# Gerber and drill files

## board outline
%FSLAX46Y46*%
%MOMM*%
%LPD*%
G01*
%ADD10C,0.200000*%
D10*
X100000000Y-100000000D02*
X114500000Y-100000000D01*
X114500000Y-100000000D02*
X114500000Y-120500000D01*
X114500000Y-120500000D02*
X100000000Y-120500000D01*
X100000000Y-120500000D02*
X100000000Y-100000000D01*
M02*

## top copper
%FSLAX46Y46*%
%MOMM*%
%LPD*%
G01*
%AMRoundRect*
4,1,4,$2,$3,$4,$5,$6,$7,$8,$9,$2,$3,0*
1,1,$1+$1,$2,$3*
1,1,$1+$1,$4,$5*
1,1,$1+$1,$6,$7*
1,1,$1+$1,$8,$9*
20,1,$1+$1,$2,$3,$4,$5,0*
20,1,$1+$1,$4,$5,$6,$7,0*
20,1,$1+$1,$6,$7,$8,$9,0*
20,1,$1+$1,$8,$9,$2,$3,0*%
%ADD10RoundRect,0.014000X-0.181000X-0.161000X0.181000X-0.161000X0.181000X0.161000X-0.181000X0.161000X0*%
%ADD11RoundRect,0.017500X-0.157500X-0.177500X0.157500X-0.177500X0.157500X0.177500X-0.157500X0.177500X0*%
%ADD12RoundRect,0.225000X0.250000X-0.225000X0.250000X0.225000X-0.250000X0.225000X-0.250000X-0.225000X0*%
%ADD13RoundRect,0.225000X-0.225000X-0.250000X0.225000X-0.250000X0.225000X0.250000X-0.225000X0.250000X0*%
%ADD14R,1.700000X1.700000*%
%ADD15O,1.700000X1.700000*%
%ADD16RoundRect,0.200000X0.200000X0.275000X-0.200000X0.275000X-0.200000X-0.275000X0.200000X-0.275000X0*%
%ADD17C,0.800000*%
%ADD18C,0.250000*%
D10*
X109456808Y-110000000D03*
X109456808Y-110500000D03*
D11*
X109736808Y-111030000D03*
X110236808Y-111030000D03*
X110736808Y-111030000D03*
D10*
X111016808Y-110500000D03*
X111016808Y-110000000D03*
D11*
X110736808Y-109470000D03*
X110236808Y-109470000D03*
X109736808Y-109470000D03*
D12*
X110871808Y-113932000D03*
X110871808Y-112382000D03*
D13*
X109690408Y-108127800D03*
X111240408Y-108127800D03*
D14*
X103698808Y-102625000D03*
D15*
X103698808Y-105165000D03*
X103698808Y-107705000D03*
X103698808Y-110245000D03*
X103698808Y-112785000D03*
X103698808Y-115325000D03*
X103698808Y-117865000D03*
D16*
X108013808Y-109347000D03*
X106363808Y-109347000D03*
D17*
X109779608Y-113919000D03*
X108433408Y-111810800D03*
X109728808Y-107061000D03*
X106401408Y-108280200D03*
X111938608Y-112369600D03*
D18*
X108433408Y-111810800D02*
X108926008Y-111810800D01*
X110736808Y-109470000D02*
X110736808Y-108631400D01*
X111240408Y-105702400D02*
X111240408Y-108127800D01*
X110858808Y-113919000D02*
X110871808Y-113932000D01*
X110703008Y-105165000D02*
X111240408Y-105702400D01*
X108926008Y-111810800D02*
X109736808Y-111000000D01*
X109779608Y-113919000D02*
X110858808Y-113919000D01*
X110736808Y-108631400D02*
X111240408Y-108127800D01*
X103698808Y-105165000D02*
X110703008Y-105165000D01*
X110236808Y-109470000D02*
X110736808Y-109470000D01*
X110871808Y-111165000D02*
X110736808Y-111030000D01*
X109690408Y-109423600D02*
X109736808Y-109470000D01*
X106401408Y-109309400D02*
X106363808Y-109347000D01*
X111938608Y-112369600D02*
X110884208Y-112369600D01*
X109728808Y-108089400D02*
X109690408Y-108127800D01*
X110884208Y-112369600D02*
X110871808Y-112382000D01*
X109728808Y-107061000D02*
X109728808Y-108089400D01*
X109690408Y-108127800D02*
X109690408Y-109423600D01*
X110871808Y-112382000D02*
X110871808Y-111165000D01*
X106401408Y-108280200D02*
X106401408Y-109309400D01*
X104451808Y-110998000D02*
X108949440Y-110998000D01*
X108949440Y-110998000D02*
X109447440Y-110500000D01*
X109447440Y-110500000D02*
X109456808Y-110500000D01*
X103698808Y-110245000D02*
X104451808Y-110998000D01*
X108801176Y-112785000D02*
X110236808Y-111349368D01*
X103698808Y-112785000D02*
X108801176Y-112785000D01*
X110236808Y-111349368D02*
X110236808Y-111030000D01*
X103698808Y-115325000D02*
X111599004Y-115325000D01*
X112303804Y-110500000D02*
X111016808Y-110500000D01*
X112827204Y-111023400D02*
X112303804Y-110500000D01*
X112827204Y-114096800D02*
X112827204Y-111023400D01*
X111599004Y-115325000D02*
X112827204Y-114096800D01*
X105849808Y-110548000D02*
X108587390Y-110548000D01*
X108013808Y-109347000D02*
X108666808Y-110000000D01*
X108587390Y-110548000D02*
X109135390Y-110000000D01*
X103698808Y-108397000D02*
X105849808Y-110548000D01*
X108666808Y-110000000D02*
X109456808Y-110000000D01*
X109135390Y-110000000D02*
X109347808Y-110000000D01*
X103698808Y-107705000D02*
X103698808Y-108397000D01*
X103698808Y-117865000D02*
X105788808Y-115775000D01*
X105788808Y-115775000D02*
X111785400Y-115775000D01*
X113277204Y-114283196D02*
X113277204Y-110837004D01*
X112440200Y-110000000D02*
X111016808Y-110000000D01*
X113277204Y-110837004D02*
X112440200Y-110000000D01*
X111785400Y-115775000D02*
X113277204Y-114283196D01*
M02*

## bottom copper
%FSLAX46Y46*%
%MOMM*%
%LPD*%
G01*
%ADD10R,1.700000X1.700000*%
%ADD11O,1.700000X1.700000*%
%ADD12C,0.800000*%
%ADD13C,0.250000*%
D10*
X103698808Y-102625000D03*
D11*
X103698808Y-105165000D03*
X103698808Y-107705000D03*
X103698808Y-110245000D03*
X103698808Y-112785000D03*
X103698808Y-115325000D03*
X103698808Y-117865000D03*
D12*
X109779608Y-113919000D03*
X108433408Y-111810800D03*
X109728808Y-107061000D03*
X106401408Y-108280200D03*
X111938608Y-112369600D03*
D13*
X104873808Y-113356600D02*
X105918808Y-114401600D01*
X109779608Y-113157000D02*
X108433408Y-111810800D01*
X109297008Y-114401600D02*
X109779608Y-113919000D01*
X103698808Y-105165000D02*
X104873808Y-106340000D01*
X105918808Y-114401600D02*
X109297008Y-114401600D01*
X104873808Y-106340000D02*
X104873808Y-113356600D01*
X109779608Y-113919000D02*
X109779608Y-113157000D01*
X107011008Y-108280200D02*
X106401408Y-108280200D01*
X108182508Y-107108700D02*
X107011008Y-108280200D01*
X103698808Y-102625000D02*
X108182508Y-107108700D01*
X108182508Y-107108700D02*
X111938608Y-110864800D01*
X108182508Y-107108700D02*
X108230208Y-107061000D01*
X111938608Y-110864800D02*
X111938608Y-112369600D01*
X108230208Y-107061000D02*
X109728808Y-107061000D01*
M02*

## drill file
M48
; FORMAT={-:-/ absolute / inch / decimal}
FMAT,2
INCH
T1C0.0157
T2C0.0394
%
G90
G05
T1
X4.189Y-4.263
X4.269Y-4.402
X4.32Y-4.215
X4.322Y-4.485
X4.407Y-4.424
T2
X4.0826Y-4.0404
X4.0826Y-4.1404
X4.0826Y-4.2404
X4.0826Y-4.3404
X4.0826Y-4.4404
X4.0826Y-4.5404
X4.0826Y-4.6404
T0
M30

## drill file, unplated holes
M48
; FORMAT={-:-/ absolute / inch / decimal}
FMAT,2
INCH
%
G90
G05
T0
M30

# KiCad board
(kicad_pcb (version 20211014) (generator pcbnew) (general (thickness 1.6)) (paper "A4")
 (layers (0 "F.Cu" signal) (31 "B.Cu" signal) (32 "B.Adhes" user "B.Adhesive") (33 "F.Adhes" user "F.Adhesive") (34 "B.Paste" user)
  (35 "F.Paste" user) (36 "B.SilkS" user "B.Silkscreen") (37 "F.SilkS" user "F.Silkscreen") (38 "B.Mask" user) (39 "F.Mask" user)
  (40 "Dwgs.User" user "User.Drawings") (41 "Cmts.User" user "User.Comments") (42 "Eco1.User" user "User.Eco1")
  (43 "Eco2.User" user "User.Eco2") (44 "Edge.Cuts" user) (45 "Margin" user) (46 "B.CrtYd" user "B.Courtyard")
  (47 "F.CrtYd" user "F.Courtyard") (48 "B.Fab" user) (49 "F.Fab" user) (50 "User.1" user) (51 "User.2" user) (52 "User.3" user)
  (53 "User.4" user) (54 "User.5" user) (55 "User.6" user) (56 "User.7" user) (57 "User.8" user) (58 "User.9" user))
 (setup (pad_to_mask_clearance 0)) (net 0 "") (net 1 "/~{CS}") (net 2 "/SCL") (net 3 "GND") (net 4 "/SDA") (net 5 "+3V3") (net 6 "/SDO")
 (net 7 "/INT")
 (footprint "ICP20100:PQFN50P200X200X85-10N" (layer "F.Cu") (at 110.236808 110.25)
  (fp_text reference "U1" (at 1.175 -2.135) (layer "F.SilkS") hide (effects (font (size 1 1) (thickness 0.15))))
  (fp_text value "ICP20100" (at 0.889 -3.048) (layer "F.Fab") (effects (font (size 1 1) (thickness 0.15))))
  (pad "1" smd roundrect locked (at -0.78 -0.25) (size 0.39 0.35) (layers "F.Cu" "F.Paste" "F.Mask") (roundrect_rratio 0.04)
   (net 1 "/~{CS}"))
  (pad "2" smd roundrect locked (at -0.78 0.25) (size 0.39 0.35) (layers "F.Cu" "F.Paste" "F.Mask") (roundrect_rratio 0.04) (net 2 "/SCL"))
  (pad "3" smd roundrect locked (at -0.5 0.78) (size 0.35 0.39) (layers "F.Cu" "F.Paste" "F.Mask") (roundrect_rratio 0.05) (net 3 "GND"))
  (pad "4" smd roundrect locked (at 0 0.78) (size 0.35 0.39) (layers "F.Cu" "F.Paste" "F.Mask") (roundrect_rratio 0.05) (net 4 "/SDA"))
  (pad "5" smd roundrect locked (at 0.5 0.78) (size 0.35 0.39) (layers "F.Cu" "F.Paste" "F.Mask") (roundrect_rratio 0.05) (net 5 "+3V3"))
  (pad "6" smd roundrect locked (at 0.78 0.25) (size 0.39 0.35) (layers "F.Cu" "F.Paste" "F.Mask") (roundrect_rratio 0.04) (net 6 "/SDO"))
  (pad "7" smd roundrect locked (at 0.78 -0.25) (size 0.39 0.35) (layers "F.Cu" "F.Paste" "F.Mask") (roundrect_rratio 0.04) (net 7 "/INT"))
  (pad "8" smd roundrect locked (at 0.5 -0.78) (size 0.35 0.39) (layers "F.Cu" "F.Paste" "F.Mask") (roundrect_rratio 0.05) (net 3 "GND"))
  (pad "9" smd roundrect locked (at 0 -0.78) (size 0.35 0.39) (layers "F.Cu" "F.Paste" "F.Mask") (roundrect_rratio 0.05) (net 3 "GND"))
  (pad "10" smd roundrect locked (at -0.5 -0.78) (size 0.35 0.39) (layers "F.Cu" "F.Paste" "F.Mask") (roundrect_rratio 0.05) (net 5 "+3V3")))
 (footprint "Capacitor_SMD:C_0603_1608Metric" (layer "F.Cu") (at 110.871808 113.157 90)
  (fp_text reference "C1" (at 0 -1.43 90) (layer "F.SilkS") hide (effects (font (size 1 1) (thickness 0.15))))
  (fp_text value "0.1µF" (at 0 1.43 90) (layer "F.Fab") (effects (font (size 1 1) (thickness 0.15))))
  (pad "1" smd roundrect (at -0.775 0 90) (size 0.9 0.95) (layers "F.Cu" "F.Paste" "F.Mask") (roundrect_rratio 0.25) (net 3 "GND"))
  (pad "2" smd roundrect (at 0.775 0 90) (size 0.9 0.95) (layers "F.Cu" "F.Paste" "F.Mask") (roundrect_rratio 0.25) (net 5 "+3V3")))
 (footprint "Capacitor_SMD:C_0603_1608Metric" (layer "F.Cu") (at 110.465408 108.1278)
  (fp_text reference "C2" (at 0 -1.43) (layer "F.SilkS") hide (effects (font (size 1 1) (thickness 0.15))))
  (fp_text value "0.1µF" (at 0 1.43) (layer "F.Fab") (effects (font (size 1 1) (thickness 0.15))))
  (pad "1" smd roundrect (at -0.775 0) (size 0.9 0.95) (layers "F.Cu" "F.Paste" "F.Mask") (roundrect_rratio 0.25) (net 5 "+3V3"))
  (pad "2" smd roundrect (at 0.775 0) (size 0.9 0.95) (layers "F.Cu" "F.Paste" "F.Mask") (roundrect_rratio 0.25) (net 3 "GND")))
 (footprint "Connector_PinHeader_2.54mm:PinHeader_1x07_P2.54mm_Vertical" (layer "F.Cu") (at 103.698808 102.625)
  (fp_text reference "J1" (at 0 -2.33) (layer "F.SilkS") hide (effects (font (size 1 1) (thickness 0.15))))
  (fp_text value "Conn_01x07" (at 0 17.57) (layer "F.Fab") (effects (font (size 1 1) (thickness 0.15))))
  (pad "1" thru_hole rect (at 0 0) (size 1.7 1.7) (drill 1) (layers *.Cu *.Mask) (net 5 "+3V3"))
  (pad "2" thru_hole oval (at 0 2.54) (size 1.7 1.7) (drill 1) (layers *.Cu *.Mask) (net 3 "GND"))
  (pad "3" thru_hole oval (at 0 5.08) (size 1.7 1.7) (drill 1) (layers *.Cu *.Mask) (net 1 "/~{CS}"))
  (pad "4" thru_hole oval (at 0 7.62) (size 1.7 1.7) (drill 1) (layers *.Cu *.Mask) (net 2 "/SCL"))
  (pad "5" thru_hole oval (at 0 10.16) (size 1.7 1.7) (drill 1) (layers *.Cu *.Mask) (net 4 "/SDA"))
  (pad "6" thru_hole oval (at 0 12.7) (size 1.7 1.7) (drill 1) (layers *.Cu *.Mask) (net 6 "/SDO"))
  (pad "7" thru_hole oval (at 0 15.24) (size 1.7 1.7) (drill 1) (layers *.Cu *.Mask) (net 7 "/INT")))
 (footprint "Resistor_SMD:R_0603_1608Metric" (layer "F.Cu") (at 107.188808 109.347 180)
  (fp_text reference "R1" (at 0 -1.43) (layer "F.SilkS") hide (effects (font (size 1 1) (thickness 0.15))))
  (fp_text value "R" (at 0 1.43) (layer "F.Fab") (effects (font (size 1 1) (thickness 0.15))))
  (pad "1" smd roundrect (at -0.825 0 180) (size 0.8 0.95) (layers "F.Cu" "F.Paste" "F.Mask") (roundrect_rratio 0.25) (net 1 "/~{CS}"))
  (pad "2" smd roundrect (at 0.825 0 180) (size 0.8 0.95) (layers "F.Cu" "F.Paste" "F.Mask") (roundrect_rratio 0.25) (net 5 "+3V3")))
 (gr_rect (start 100 100) (end 114.5 120.5) (layer "Edge.Cuts") (width 0.2) (fill none))
 (segment (start 108.433408 111.8108) (end 108.926008 111.8108) (width 0.25) (layer "F.Cu") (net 3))
 (segment (start 110.736808 109.47) (end 110.736808 108.6314) (width 0.25) (layer "F.Cu") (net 3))
 (segment (start 111.240408 105.7024) (end 111.240408 108.1278) (width 0.25) (layer "F.Cu") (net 3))
 (segment (start 110.858808 113.919) (end 110.871808 113.932) (width 0.25) (layer "F.Cu") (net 3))
 (segment (start 110.703008 105.165) (end 111.240408 105.7024) (width 0.25) (layer "F.Cu") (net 3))
 (segment (start 108.926008 111.8108) (end 109.736808 111) (width 0.25) (layer "F.Cu") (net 3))
 (segment (start 109.779608 113.919) (end 110.858808 113.919) (width 0.25) (layer "F.Cu") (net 3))
 (segment (start 110.736808 108.6314) (end 111.240408 108.1278) (width 0.25) (layer "F.Cu") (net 3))
 (segment (start 103.698808 105.165) (end 110.703008 105.165) (width 0.25) (layer "F.Cu") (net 3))
 (segment (start 110.236808 109.47) (end 110.736808 109.47) (width 0.25) (layer "F.Cu") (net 3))
 (via (at 109.779608 113.919) (size 0.8) (drill 0.4) (layers "F.Cu" "B.Cu") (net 3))
 (via (at 108.433408 111.8108) (size 0.8) (drill 0.4) (layers "F.Cu" "B.Cu") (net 3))
 (segment (start 104.873808 113.3566) (end 105.918808 114.4016) (width 0.25) (layer "B.Cu") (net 3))
 (segment (start 109.779608 113.157) (end 108.433408 111.8108) (width 0.25) (layer "B.Cu") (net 3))
 (segment (start 109.297008 114.4016) (end 109.779608 113.919) (width 0.25) (layer "B.Cu") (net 3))
 (segment (start 103.698808 105.165) (end 104.873808 106.34) (width 0.25) (layer "B.Cu") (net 3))
 (segment (start 105.918808 114.4016) (end 109.297008 114.4016) (width 0.25) (layer "B.Cu") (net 3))
 (segment (start 104.873808 106.34) (end 104.873808 113.3566) (width 0.25) (layer "B.Cu") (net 3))
 (segment (start 109.779608 113.919) (end 109.779608 113.157) (width 0.25) (layer "B.Cu") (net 3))
 (segment (start 110.871808 111.165) (end 110.736808 111.03) (width 0.25) (layer "F.Cu") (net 5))
 (segment (start 109.690408 109.4236) (end 109.736808 109.47) (width 0.25) (layer "F.Cu") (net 5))
 (segment (start 106.401408 109.3094) (end 106.363808 109.347) (width 0.25) (layer "F.Cu") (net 5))
 (segment (start 111.938608 112.3696) (end 110.884208 112.3696) (width 0.25) (layer "F.Cu") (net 5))
 (segment (start 109.728808 108.0894) (end 109.690408 108.1278) (width 0.25) (layer "F.Cu") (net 5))
 (segment (start 110.884208 112.3696) (end 110.871808 112.382) (width 0.25) (layer "F.Cu") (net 5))
 (segment (start 109.728808 107.061) (end 109.728808 108.0894) (width 0.25) (layer "F.Cu") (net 5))
 (segment (start 109.690408 108.1278) (end 109.690408 109.4236) (width 0.25) (layer "F.Cu") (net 5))
 (segment (start 110.871808 112.382) (end 110.871808 111.165) (width 0.25) (layer "F.Cu") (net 5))
 (segment (start 106.401408 108.2802) (end 106.401408 109.3094) (width 0.25) (layer "F.Cu") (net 5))
 (via (at 109.728808 107.061) (size 0.8) (drill 0.4) (layers "F.Cu" "B.Cu") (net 5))
 (via (at 106.401408 108.2802) (size 0.8) (drill 0.4) (layers "F.Cu" "B.Cu") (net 5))
 (via (at 111.938608 112.3696) (size 0.8) (drill 0.4) (layers "F.Cu" "B.Cu") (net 5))
 (segment (start 107.011008 108.2802) (end 106.401408 108.2802) (width 0.25) (layer "B.Cu") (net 5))
 (segment (start 108.182508 107.1087) (end 107.011008 108.2802) (width 0.25) (layer "B.Cu") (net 5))
 (segment (start 103.698808 102.625) (end 108.182508 107.1087) (width 0.25) (layer "B.Cu") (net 5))
 (segment (start 108.182508 107.1087) (end 111.938608 110.8648) (width 0.25) (layer "B.Cu") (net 5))
 (segment (start 108.182508 107.1087) (end 108.230208 107.061) (width 0.25) (layer "B.Cu") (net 5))
 (segment (start 111.938608 110.8648) (end 111.938608 112.3696) (width 0.25) (layer "B.Cu") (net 5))
 (segment (start 108.230208 107.061) (end 109.728808 107.061) (width 0.25) (layer "B.Cu") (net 5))
 (segment (start 104.451808 110.998) (end 108.94944 110.998) (width 0.25) (layer "F.Cu") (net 2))
 (segment (start 108.94944 110.998) (end 109.44744 110.5) (width 0.25) (layer "F.Cu") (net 2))
 (segment (start 109.44744 110.5) (end 109.456808 110.5) (width 0.25) (layer "F.Cu") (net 2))
 (segment (start 103.698808 110.245) (end 104.451808 110.998) (width 0.25) (layer "F.Cu") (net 2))
 (segment (start 108.801176 112.785) (end 110.236808 111.349368) (width 0.25) (layer "F.Cu") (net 4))
 (segment (start 103.698808 112.785) (end 108.801176 112.785) (width 0.25) (layer "F.Cu") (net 4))
 (segment (start 110.236808 111.349368) (end 110.236808 111.03) (width 0.25) (layer "F.Cu") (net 4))
 (segment (start 103.698808 115.325) (end 111.599004 115.325) (width 0.25) (layer "F.Cu") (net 6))
 (segment (start 112.303804 110.5) (end 111.016808 110.5) (width 0.25) (layer "F.Cu") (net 6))
 (segment (start 112.827204 111.0234) (end 112.303804 110.5) (width 0.25) (layer "F.Cu") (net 6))
 (segment (start 112.827204 114.0968) (end 112.827204 111.0234) (width 0.25) (layer "F.Cu") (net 6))
 (segment (start 111.599004 115.325) (end 112.827204 114.0968) (width 0.25) (layer "F.Cu") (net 6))
 (segment (start 105.849808 110.548) (end 108.58739 110.548) (width 0.25) (layer "F.Cu") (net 1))
 (segment (start 108.013808 109.347) (end 108.666808 110) (width 0.25) (layer "F.Cu") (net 1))
 (segment (start 108.58739 110.548) (end 109.13539 110) (width 0.25) (layer "F.Cu") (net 1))
 (segment (start 103.698808 108.397) (end 105.849808 110.548) (width 0.25) (layer "F.Cu") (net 1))
 (segment (start 108.666808 110) (end 109.456808 110) (width 0.25) (layer "F.Cu") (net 1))
 (segment (start 109.13539 110) (end 109.347808 110) (width 0.25) (layer "F.Cu") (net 1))
 (segment (start 103.698808 107.705) (end 103.698808 108.397) (width 0.25) (layer "F.Cu") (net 1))
 (segment (start 103.698808 117.865) (end 105.788808 115.775) (width 0.25) (layer "F.Cu") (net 7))
 (segment (start 105.788808 115.775) (end 111.7854 115.775) (width 0.25) (layer "F.Cu") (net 7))
 (segment (start 113.277204 114.283196) (end 113.277204 110.837004) (width 0.25) (layer "F.Cu") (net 7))
 (segment (start 112.4402 110) (end 111.016808 110) (width 0.25) (layer "F.Cu") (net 7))
 (segment (start 113.277204 110.837004) (end 112.4402 110) (width 0.25) (layer "F.Cu") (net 7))
 (segment (start 111.7854 115.775) (end 113.277204 114.283196) (width 0.25) (layer "F.Cu") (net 7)))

